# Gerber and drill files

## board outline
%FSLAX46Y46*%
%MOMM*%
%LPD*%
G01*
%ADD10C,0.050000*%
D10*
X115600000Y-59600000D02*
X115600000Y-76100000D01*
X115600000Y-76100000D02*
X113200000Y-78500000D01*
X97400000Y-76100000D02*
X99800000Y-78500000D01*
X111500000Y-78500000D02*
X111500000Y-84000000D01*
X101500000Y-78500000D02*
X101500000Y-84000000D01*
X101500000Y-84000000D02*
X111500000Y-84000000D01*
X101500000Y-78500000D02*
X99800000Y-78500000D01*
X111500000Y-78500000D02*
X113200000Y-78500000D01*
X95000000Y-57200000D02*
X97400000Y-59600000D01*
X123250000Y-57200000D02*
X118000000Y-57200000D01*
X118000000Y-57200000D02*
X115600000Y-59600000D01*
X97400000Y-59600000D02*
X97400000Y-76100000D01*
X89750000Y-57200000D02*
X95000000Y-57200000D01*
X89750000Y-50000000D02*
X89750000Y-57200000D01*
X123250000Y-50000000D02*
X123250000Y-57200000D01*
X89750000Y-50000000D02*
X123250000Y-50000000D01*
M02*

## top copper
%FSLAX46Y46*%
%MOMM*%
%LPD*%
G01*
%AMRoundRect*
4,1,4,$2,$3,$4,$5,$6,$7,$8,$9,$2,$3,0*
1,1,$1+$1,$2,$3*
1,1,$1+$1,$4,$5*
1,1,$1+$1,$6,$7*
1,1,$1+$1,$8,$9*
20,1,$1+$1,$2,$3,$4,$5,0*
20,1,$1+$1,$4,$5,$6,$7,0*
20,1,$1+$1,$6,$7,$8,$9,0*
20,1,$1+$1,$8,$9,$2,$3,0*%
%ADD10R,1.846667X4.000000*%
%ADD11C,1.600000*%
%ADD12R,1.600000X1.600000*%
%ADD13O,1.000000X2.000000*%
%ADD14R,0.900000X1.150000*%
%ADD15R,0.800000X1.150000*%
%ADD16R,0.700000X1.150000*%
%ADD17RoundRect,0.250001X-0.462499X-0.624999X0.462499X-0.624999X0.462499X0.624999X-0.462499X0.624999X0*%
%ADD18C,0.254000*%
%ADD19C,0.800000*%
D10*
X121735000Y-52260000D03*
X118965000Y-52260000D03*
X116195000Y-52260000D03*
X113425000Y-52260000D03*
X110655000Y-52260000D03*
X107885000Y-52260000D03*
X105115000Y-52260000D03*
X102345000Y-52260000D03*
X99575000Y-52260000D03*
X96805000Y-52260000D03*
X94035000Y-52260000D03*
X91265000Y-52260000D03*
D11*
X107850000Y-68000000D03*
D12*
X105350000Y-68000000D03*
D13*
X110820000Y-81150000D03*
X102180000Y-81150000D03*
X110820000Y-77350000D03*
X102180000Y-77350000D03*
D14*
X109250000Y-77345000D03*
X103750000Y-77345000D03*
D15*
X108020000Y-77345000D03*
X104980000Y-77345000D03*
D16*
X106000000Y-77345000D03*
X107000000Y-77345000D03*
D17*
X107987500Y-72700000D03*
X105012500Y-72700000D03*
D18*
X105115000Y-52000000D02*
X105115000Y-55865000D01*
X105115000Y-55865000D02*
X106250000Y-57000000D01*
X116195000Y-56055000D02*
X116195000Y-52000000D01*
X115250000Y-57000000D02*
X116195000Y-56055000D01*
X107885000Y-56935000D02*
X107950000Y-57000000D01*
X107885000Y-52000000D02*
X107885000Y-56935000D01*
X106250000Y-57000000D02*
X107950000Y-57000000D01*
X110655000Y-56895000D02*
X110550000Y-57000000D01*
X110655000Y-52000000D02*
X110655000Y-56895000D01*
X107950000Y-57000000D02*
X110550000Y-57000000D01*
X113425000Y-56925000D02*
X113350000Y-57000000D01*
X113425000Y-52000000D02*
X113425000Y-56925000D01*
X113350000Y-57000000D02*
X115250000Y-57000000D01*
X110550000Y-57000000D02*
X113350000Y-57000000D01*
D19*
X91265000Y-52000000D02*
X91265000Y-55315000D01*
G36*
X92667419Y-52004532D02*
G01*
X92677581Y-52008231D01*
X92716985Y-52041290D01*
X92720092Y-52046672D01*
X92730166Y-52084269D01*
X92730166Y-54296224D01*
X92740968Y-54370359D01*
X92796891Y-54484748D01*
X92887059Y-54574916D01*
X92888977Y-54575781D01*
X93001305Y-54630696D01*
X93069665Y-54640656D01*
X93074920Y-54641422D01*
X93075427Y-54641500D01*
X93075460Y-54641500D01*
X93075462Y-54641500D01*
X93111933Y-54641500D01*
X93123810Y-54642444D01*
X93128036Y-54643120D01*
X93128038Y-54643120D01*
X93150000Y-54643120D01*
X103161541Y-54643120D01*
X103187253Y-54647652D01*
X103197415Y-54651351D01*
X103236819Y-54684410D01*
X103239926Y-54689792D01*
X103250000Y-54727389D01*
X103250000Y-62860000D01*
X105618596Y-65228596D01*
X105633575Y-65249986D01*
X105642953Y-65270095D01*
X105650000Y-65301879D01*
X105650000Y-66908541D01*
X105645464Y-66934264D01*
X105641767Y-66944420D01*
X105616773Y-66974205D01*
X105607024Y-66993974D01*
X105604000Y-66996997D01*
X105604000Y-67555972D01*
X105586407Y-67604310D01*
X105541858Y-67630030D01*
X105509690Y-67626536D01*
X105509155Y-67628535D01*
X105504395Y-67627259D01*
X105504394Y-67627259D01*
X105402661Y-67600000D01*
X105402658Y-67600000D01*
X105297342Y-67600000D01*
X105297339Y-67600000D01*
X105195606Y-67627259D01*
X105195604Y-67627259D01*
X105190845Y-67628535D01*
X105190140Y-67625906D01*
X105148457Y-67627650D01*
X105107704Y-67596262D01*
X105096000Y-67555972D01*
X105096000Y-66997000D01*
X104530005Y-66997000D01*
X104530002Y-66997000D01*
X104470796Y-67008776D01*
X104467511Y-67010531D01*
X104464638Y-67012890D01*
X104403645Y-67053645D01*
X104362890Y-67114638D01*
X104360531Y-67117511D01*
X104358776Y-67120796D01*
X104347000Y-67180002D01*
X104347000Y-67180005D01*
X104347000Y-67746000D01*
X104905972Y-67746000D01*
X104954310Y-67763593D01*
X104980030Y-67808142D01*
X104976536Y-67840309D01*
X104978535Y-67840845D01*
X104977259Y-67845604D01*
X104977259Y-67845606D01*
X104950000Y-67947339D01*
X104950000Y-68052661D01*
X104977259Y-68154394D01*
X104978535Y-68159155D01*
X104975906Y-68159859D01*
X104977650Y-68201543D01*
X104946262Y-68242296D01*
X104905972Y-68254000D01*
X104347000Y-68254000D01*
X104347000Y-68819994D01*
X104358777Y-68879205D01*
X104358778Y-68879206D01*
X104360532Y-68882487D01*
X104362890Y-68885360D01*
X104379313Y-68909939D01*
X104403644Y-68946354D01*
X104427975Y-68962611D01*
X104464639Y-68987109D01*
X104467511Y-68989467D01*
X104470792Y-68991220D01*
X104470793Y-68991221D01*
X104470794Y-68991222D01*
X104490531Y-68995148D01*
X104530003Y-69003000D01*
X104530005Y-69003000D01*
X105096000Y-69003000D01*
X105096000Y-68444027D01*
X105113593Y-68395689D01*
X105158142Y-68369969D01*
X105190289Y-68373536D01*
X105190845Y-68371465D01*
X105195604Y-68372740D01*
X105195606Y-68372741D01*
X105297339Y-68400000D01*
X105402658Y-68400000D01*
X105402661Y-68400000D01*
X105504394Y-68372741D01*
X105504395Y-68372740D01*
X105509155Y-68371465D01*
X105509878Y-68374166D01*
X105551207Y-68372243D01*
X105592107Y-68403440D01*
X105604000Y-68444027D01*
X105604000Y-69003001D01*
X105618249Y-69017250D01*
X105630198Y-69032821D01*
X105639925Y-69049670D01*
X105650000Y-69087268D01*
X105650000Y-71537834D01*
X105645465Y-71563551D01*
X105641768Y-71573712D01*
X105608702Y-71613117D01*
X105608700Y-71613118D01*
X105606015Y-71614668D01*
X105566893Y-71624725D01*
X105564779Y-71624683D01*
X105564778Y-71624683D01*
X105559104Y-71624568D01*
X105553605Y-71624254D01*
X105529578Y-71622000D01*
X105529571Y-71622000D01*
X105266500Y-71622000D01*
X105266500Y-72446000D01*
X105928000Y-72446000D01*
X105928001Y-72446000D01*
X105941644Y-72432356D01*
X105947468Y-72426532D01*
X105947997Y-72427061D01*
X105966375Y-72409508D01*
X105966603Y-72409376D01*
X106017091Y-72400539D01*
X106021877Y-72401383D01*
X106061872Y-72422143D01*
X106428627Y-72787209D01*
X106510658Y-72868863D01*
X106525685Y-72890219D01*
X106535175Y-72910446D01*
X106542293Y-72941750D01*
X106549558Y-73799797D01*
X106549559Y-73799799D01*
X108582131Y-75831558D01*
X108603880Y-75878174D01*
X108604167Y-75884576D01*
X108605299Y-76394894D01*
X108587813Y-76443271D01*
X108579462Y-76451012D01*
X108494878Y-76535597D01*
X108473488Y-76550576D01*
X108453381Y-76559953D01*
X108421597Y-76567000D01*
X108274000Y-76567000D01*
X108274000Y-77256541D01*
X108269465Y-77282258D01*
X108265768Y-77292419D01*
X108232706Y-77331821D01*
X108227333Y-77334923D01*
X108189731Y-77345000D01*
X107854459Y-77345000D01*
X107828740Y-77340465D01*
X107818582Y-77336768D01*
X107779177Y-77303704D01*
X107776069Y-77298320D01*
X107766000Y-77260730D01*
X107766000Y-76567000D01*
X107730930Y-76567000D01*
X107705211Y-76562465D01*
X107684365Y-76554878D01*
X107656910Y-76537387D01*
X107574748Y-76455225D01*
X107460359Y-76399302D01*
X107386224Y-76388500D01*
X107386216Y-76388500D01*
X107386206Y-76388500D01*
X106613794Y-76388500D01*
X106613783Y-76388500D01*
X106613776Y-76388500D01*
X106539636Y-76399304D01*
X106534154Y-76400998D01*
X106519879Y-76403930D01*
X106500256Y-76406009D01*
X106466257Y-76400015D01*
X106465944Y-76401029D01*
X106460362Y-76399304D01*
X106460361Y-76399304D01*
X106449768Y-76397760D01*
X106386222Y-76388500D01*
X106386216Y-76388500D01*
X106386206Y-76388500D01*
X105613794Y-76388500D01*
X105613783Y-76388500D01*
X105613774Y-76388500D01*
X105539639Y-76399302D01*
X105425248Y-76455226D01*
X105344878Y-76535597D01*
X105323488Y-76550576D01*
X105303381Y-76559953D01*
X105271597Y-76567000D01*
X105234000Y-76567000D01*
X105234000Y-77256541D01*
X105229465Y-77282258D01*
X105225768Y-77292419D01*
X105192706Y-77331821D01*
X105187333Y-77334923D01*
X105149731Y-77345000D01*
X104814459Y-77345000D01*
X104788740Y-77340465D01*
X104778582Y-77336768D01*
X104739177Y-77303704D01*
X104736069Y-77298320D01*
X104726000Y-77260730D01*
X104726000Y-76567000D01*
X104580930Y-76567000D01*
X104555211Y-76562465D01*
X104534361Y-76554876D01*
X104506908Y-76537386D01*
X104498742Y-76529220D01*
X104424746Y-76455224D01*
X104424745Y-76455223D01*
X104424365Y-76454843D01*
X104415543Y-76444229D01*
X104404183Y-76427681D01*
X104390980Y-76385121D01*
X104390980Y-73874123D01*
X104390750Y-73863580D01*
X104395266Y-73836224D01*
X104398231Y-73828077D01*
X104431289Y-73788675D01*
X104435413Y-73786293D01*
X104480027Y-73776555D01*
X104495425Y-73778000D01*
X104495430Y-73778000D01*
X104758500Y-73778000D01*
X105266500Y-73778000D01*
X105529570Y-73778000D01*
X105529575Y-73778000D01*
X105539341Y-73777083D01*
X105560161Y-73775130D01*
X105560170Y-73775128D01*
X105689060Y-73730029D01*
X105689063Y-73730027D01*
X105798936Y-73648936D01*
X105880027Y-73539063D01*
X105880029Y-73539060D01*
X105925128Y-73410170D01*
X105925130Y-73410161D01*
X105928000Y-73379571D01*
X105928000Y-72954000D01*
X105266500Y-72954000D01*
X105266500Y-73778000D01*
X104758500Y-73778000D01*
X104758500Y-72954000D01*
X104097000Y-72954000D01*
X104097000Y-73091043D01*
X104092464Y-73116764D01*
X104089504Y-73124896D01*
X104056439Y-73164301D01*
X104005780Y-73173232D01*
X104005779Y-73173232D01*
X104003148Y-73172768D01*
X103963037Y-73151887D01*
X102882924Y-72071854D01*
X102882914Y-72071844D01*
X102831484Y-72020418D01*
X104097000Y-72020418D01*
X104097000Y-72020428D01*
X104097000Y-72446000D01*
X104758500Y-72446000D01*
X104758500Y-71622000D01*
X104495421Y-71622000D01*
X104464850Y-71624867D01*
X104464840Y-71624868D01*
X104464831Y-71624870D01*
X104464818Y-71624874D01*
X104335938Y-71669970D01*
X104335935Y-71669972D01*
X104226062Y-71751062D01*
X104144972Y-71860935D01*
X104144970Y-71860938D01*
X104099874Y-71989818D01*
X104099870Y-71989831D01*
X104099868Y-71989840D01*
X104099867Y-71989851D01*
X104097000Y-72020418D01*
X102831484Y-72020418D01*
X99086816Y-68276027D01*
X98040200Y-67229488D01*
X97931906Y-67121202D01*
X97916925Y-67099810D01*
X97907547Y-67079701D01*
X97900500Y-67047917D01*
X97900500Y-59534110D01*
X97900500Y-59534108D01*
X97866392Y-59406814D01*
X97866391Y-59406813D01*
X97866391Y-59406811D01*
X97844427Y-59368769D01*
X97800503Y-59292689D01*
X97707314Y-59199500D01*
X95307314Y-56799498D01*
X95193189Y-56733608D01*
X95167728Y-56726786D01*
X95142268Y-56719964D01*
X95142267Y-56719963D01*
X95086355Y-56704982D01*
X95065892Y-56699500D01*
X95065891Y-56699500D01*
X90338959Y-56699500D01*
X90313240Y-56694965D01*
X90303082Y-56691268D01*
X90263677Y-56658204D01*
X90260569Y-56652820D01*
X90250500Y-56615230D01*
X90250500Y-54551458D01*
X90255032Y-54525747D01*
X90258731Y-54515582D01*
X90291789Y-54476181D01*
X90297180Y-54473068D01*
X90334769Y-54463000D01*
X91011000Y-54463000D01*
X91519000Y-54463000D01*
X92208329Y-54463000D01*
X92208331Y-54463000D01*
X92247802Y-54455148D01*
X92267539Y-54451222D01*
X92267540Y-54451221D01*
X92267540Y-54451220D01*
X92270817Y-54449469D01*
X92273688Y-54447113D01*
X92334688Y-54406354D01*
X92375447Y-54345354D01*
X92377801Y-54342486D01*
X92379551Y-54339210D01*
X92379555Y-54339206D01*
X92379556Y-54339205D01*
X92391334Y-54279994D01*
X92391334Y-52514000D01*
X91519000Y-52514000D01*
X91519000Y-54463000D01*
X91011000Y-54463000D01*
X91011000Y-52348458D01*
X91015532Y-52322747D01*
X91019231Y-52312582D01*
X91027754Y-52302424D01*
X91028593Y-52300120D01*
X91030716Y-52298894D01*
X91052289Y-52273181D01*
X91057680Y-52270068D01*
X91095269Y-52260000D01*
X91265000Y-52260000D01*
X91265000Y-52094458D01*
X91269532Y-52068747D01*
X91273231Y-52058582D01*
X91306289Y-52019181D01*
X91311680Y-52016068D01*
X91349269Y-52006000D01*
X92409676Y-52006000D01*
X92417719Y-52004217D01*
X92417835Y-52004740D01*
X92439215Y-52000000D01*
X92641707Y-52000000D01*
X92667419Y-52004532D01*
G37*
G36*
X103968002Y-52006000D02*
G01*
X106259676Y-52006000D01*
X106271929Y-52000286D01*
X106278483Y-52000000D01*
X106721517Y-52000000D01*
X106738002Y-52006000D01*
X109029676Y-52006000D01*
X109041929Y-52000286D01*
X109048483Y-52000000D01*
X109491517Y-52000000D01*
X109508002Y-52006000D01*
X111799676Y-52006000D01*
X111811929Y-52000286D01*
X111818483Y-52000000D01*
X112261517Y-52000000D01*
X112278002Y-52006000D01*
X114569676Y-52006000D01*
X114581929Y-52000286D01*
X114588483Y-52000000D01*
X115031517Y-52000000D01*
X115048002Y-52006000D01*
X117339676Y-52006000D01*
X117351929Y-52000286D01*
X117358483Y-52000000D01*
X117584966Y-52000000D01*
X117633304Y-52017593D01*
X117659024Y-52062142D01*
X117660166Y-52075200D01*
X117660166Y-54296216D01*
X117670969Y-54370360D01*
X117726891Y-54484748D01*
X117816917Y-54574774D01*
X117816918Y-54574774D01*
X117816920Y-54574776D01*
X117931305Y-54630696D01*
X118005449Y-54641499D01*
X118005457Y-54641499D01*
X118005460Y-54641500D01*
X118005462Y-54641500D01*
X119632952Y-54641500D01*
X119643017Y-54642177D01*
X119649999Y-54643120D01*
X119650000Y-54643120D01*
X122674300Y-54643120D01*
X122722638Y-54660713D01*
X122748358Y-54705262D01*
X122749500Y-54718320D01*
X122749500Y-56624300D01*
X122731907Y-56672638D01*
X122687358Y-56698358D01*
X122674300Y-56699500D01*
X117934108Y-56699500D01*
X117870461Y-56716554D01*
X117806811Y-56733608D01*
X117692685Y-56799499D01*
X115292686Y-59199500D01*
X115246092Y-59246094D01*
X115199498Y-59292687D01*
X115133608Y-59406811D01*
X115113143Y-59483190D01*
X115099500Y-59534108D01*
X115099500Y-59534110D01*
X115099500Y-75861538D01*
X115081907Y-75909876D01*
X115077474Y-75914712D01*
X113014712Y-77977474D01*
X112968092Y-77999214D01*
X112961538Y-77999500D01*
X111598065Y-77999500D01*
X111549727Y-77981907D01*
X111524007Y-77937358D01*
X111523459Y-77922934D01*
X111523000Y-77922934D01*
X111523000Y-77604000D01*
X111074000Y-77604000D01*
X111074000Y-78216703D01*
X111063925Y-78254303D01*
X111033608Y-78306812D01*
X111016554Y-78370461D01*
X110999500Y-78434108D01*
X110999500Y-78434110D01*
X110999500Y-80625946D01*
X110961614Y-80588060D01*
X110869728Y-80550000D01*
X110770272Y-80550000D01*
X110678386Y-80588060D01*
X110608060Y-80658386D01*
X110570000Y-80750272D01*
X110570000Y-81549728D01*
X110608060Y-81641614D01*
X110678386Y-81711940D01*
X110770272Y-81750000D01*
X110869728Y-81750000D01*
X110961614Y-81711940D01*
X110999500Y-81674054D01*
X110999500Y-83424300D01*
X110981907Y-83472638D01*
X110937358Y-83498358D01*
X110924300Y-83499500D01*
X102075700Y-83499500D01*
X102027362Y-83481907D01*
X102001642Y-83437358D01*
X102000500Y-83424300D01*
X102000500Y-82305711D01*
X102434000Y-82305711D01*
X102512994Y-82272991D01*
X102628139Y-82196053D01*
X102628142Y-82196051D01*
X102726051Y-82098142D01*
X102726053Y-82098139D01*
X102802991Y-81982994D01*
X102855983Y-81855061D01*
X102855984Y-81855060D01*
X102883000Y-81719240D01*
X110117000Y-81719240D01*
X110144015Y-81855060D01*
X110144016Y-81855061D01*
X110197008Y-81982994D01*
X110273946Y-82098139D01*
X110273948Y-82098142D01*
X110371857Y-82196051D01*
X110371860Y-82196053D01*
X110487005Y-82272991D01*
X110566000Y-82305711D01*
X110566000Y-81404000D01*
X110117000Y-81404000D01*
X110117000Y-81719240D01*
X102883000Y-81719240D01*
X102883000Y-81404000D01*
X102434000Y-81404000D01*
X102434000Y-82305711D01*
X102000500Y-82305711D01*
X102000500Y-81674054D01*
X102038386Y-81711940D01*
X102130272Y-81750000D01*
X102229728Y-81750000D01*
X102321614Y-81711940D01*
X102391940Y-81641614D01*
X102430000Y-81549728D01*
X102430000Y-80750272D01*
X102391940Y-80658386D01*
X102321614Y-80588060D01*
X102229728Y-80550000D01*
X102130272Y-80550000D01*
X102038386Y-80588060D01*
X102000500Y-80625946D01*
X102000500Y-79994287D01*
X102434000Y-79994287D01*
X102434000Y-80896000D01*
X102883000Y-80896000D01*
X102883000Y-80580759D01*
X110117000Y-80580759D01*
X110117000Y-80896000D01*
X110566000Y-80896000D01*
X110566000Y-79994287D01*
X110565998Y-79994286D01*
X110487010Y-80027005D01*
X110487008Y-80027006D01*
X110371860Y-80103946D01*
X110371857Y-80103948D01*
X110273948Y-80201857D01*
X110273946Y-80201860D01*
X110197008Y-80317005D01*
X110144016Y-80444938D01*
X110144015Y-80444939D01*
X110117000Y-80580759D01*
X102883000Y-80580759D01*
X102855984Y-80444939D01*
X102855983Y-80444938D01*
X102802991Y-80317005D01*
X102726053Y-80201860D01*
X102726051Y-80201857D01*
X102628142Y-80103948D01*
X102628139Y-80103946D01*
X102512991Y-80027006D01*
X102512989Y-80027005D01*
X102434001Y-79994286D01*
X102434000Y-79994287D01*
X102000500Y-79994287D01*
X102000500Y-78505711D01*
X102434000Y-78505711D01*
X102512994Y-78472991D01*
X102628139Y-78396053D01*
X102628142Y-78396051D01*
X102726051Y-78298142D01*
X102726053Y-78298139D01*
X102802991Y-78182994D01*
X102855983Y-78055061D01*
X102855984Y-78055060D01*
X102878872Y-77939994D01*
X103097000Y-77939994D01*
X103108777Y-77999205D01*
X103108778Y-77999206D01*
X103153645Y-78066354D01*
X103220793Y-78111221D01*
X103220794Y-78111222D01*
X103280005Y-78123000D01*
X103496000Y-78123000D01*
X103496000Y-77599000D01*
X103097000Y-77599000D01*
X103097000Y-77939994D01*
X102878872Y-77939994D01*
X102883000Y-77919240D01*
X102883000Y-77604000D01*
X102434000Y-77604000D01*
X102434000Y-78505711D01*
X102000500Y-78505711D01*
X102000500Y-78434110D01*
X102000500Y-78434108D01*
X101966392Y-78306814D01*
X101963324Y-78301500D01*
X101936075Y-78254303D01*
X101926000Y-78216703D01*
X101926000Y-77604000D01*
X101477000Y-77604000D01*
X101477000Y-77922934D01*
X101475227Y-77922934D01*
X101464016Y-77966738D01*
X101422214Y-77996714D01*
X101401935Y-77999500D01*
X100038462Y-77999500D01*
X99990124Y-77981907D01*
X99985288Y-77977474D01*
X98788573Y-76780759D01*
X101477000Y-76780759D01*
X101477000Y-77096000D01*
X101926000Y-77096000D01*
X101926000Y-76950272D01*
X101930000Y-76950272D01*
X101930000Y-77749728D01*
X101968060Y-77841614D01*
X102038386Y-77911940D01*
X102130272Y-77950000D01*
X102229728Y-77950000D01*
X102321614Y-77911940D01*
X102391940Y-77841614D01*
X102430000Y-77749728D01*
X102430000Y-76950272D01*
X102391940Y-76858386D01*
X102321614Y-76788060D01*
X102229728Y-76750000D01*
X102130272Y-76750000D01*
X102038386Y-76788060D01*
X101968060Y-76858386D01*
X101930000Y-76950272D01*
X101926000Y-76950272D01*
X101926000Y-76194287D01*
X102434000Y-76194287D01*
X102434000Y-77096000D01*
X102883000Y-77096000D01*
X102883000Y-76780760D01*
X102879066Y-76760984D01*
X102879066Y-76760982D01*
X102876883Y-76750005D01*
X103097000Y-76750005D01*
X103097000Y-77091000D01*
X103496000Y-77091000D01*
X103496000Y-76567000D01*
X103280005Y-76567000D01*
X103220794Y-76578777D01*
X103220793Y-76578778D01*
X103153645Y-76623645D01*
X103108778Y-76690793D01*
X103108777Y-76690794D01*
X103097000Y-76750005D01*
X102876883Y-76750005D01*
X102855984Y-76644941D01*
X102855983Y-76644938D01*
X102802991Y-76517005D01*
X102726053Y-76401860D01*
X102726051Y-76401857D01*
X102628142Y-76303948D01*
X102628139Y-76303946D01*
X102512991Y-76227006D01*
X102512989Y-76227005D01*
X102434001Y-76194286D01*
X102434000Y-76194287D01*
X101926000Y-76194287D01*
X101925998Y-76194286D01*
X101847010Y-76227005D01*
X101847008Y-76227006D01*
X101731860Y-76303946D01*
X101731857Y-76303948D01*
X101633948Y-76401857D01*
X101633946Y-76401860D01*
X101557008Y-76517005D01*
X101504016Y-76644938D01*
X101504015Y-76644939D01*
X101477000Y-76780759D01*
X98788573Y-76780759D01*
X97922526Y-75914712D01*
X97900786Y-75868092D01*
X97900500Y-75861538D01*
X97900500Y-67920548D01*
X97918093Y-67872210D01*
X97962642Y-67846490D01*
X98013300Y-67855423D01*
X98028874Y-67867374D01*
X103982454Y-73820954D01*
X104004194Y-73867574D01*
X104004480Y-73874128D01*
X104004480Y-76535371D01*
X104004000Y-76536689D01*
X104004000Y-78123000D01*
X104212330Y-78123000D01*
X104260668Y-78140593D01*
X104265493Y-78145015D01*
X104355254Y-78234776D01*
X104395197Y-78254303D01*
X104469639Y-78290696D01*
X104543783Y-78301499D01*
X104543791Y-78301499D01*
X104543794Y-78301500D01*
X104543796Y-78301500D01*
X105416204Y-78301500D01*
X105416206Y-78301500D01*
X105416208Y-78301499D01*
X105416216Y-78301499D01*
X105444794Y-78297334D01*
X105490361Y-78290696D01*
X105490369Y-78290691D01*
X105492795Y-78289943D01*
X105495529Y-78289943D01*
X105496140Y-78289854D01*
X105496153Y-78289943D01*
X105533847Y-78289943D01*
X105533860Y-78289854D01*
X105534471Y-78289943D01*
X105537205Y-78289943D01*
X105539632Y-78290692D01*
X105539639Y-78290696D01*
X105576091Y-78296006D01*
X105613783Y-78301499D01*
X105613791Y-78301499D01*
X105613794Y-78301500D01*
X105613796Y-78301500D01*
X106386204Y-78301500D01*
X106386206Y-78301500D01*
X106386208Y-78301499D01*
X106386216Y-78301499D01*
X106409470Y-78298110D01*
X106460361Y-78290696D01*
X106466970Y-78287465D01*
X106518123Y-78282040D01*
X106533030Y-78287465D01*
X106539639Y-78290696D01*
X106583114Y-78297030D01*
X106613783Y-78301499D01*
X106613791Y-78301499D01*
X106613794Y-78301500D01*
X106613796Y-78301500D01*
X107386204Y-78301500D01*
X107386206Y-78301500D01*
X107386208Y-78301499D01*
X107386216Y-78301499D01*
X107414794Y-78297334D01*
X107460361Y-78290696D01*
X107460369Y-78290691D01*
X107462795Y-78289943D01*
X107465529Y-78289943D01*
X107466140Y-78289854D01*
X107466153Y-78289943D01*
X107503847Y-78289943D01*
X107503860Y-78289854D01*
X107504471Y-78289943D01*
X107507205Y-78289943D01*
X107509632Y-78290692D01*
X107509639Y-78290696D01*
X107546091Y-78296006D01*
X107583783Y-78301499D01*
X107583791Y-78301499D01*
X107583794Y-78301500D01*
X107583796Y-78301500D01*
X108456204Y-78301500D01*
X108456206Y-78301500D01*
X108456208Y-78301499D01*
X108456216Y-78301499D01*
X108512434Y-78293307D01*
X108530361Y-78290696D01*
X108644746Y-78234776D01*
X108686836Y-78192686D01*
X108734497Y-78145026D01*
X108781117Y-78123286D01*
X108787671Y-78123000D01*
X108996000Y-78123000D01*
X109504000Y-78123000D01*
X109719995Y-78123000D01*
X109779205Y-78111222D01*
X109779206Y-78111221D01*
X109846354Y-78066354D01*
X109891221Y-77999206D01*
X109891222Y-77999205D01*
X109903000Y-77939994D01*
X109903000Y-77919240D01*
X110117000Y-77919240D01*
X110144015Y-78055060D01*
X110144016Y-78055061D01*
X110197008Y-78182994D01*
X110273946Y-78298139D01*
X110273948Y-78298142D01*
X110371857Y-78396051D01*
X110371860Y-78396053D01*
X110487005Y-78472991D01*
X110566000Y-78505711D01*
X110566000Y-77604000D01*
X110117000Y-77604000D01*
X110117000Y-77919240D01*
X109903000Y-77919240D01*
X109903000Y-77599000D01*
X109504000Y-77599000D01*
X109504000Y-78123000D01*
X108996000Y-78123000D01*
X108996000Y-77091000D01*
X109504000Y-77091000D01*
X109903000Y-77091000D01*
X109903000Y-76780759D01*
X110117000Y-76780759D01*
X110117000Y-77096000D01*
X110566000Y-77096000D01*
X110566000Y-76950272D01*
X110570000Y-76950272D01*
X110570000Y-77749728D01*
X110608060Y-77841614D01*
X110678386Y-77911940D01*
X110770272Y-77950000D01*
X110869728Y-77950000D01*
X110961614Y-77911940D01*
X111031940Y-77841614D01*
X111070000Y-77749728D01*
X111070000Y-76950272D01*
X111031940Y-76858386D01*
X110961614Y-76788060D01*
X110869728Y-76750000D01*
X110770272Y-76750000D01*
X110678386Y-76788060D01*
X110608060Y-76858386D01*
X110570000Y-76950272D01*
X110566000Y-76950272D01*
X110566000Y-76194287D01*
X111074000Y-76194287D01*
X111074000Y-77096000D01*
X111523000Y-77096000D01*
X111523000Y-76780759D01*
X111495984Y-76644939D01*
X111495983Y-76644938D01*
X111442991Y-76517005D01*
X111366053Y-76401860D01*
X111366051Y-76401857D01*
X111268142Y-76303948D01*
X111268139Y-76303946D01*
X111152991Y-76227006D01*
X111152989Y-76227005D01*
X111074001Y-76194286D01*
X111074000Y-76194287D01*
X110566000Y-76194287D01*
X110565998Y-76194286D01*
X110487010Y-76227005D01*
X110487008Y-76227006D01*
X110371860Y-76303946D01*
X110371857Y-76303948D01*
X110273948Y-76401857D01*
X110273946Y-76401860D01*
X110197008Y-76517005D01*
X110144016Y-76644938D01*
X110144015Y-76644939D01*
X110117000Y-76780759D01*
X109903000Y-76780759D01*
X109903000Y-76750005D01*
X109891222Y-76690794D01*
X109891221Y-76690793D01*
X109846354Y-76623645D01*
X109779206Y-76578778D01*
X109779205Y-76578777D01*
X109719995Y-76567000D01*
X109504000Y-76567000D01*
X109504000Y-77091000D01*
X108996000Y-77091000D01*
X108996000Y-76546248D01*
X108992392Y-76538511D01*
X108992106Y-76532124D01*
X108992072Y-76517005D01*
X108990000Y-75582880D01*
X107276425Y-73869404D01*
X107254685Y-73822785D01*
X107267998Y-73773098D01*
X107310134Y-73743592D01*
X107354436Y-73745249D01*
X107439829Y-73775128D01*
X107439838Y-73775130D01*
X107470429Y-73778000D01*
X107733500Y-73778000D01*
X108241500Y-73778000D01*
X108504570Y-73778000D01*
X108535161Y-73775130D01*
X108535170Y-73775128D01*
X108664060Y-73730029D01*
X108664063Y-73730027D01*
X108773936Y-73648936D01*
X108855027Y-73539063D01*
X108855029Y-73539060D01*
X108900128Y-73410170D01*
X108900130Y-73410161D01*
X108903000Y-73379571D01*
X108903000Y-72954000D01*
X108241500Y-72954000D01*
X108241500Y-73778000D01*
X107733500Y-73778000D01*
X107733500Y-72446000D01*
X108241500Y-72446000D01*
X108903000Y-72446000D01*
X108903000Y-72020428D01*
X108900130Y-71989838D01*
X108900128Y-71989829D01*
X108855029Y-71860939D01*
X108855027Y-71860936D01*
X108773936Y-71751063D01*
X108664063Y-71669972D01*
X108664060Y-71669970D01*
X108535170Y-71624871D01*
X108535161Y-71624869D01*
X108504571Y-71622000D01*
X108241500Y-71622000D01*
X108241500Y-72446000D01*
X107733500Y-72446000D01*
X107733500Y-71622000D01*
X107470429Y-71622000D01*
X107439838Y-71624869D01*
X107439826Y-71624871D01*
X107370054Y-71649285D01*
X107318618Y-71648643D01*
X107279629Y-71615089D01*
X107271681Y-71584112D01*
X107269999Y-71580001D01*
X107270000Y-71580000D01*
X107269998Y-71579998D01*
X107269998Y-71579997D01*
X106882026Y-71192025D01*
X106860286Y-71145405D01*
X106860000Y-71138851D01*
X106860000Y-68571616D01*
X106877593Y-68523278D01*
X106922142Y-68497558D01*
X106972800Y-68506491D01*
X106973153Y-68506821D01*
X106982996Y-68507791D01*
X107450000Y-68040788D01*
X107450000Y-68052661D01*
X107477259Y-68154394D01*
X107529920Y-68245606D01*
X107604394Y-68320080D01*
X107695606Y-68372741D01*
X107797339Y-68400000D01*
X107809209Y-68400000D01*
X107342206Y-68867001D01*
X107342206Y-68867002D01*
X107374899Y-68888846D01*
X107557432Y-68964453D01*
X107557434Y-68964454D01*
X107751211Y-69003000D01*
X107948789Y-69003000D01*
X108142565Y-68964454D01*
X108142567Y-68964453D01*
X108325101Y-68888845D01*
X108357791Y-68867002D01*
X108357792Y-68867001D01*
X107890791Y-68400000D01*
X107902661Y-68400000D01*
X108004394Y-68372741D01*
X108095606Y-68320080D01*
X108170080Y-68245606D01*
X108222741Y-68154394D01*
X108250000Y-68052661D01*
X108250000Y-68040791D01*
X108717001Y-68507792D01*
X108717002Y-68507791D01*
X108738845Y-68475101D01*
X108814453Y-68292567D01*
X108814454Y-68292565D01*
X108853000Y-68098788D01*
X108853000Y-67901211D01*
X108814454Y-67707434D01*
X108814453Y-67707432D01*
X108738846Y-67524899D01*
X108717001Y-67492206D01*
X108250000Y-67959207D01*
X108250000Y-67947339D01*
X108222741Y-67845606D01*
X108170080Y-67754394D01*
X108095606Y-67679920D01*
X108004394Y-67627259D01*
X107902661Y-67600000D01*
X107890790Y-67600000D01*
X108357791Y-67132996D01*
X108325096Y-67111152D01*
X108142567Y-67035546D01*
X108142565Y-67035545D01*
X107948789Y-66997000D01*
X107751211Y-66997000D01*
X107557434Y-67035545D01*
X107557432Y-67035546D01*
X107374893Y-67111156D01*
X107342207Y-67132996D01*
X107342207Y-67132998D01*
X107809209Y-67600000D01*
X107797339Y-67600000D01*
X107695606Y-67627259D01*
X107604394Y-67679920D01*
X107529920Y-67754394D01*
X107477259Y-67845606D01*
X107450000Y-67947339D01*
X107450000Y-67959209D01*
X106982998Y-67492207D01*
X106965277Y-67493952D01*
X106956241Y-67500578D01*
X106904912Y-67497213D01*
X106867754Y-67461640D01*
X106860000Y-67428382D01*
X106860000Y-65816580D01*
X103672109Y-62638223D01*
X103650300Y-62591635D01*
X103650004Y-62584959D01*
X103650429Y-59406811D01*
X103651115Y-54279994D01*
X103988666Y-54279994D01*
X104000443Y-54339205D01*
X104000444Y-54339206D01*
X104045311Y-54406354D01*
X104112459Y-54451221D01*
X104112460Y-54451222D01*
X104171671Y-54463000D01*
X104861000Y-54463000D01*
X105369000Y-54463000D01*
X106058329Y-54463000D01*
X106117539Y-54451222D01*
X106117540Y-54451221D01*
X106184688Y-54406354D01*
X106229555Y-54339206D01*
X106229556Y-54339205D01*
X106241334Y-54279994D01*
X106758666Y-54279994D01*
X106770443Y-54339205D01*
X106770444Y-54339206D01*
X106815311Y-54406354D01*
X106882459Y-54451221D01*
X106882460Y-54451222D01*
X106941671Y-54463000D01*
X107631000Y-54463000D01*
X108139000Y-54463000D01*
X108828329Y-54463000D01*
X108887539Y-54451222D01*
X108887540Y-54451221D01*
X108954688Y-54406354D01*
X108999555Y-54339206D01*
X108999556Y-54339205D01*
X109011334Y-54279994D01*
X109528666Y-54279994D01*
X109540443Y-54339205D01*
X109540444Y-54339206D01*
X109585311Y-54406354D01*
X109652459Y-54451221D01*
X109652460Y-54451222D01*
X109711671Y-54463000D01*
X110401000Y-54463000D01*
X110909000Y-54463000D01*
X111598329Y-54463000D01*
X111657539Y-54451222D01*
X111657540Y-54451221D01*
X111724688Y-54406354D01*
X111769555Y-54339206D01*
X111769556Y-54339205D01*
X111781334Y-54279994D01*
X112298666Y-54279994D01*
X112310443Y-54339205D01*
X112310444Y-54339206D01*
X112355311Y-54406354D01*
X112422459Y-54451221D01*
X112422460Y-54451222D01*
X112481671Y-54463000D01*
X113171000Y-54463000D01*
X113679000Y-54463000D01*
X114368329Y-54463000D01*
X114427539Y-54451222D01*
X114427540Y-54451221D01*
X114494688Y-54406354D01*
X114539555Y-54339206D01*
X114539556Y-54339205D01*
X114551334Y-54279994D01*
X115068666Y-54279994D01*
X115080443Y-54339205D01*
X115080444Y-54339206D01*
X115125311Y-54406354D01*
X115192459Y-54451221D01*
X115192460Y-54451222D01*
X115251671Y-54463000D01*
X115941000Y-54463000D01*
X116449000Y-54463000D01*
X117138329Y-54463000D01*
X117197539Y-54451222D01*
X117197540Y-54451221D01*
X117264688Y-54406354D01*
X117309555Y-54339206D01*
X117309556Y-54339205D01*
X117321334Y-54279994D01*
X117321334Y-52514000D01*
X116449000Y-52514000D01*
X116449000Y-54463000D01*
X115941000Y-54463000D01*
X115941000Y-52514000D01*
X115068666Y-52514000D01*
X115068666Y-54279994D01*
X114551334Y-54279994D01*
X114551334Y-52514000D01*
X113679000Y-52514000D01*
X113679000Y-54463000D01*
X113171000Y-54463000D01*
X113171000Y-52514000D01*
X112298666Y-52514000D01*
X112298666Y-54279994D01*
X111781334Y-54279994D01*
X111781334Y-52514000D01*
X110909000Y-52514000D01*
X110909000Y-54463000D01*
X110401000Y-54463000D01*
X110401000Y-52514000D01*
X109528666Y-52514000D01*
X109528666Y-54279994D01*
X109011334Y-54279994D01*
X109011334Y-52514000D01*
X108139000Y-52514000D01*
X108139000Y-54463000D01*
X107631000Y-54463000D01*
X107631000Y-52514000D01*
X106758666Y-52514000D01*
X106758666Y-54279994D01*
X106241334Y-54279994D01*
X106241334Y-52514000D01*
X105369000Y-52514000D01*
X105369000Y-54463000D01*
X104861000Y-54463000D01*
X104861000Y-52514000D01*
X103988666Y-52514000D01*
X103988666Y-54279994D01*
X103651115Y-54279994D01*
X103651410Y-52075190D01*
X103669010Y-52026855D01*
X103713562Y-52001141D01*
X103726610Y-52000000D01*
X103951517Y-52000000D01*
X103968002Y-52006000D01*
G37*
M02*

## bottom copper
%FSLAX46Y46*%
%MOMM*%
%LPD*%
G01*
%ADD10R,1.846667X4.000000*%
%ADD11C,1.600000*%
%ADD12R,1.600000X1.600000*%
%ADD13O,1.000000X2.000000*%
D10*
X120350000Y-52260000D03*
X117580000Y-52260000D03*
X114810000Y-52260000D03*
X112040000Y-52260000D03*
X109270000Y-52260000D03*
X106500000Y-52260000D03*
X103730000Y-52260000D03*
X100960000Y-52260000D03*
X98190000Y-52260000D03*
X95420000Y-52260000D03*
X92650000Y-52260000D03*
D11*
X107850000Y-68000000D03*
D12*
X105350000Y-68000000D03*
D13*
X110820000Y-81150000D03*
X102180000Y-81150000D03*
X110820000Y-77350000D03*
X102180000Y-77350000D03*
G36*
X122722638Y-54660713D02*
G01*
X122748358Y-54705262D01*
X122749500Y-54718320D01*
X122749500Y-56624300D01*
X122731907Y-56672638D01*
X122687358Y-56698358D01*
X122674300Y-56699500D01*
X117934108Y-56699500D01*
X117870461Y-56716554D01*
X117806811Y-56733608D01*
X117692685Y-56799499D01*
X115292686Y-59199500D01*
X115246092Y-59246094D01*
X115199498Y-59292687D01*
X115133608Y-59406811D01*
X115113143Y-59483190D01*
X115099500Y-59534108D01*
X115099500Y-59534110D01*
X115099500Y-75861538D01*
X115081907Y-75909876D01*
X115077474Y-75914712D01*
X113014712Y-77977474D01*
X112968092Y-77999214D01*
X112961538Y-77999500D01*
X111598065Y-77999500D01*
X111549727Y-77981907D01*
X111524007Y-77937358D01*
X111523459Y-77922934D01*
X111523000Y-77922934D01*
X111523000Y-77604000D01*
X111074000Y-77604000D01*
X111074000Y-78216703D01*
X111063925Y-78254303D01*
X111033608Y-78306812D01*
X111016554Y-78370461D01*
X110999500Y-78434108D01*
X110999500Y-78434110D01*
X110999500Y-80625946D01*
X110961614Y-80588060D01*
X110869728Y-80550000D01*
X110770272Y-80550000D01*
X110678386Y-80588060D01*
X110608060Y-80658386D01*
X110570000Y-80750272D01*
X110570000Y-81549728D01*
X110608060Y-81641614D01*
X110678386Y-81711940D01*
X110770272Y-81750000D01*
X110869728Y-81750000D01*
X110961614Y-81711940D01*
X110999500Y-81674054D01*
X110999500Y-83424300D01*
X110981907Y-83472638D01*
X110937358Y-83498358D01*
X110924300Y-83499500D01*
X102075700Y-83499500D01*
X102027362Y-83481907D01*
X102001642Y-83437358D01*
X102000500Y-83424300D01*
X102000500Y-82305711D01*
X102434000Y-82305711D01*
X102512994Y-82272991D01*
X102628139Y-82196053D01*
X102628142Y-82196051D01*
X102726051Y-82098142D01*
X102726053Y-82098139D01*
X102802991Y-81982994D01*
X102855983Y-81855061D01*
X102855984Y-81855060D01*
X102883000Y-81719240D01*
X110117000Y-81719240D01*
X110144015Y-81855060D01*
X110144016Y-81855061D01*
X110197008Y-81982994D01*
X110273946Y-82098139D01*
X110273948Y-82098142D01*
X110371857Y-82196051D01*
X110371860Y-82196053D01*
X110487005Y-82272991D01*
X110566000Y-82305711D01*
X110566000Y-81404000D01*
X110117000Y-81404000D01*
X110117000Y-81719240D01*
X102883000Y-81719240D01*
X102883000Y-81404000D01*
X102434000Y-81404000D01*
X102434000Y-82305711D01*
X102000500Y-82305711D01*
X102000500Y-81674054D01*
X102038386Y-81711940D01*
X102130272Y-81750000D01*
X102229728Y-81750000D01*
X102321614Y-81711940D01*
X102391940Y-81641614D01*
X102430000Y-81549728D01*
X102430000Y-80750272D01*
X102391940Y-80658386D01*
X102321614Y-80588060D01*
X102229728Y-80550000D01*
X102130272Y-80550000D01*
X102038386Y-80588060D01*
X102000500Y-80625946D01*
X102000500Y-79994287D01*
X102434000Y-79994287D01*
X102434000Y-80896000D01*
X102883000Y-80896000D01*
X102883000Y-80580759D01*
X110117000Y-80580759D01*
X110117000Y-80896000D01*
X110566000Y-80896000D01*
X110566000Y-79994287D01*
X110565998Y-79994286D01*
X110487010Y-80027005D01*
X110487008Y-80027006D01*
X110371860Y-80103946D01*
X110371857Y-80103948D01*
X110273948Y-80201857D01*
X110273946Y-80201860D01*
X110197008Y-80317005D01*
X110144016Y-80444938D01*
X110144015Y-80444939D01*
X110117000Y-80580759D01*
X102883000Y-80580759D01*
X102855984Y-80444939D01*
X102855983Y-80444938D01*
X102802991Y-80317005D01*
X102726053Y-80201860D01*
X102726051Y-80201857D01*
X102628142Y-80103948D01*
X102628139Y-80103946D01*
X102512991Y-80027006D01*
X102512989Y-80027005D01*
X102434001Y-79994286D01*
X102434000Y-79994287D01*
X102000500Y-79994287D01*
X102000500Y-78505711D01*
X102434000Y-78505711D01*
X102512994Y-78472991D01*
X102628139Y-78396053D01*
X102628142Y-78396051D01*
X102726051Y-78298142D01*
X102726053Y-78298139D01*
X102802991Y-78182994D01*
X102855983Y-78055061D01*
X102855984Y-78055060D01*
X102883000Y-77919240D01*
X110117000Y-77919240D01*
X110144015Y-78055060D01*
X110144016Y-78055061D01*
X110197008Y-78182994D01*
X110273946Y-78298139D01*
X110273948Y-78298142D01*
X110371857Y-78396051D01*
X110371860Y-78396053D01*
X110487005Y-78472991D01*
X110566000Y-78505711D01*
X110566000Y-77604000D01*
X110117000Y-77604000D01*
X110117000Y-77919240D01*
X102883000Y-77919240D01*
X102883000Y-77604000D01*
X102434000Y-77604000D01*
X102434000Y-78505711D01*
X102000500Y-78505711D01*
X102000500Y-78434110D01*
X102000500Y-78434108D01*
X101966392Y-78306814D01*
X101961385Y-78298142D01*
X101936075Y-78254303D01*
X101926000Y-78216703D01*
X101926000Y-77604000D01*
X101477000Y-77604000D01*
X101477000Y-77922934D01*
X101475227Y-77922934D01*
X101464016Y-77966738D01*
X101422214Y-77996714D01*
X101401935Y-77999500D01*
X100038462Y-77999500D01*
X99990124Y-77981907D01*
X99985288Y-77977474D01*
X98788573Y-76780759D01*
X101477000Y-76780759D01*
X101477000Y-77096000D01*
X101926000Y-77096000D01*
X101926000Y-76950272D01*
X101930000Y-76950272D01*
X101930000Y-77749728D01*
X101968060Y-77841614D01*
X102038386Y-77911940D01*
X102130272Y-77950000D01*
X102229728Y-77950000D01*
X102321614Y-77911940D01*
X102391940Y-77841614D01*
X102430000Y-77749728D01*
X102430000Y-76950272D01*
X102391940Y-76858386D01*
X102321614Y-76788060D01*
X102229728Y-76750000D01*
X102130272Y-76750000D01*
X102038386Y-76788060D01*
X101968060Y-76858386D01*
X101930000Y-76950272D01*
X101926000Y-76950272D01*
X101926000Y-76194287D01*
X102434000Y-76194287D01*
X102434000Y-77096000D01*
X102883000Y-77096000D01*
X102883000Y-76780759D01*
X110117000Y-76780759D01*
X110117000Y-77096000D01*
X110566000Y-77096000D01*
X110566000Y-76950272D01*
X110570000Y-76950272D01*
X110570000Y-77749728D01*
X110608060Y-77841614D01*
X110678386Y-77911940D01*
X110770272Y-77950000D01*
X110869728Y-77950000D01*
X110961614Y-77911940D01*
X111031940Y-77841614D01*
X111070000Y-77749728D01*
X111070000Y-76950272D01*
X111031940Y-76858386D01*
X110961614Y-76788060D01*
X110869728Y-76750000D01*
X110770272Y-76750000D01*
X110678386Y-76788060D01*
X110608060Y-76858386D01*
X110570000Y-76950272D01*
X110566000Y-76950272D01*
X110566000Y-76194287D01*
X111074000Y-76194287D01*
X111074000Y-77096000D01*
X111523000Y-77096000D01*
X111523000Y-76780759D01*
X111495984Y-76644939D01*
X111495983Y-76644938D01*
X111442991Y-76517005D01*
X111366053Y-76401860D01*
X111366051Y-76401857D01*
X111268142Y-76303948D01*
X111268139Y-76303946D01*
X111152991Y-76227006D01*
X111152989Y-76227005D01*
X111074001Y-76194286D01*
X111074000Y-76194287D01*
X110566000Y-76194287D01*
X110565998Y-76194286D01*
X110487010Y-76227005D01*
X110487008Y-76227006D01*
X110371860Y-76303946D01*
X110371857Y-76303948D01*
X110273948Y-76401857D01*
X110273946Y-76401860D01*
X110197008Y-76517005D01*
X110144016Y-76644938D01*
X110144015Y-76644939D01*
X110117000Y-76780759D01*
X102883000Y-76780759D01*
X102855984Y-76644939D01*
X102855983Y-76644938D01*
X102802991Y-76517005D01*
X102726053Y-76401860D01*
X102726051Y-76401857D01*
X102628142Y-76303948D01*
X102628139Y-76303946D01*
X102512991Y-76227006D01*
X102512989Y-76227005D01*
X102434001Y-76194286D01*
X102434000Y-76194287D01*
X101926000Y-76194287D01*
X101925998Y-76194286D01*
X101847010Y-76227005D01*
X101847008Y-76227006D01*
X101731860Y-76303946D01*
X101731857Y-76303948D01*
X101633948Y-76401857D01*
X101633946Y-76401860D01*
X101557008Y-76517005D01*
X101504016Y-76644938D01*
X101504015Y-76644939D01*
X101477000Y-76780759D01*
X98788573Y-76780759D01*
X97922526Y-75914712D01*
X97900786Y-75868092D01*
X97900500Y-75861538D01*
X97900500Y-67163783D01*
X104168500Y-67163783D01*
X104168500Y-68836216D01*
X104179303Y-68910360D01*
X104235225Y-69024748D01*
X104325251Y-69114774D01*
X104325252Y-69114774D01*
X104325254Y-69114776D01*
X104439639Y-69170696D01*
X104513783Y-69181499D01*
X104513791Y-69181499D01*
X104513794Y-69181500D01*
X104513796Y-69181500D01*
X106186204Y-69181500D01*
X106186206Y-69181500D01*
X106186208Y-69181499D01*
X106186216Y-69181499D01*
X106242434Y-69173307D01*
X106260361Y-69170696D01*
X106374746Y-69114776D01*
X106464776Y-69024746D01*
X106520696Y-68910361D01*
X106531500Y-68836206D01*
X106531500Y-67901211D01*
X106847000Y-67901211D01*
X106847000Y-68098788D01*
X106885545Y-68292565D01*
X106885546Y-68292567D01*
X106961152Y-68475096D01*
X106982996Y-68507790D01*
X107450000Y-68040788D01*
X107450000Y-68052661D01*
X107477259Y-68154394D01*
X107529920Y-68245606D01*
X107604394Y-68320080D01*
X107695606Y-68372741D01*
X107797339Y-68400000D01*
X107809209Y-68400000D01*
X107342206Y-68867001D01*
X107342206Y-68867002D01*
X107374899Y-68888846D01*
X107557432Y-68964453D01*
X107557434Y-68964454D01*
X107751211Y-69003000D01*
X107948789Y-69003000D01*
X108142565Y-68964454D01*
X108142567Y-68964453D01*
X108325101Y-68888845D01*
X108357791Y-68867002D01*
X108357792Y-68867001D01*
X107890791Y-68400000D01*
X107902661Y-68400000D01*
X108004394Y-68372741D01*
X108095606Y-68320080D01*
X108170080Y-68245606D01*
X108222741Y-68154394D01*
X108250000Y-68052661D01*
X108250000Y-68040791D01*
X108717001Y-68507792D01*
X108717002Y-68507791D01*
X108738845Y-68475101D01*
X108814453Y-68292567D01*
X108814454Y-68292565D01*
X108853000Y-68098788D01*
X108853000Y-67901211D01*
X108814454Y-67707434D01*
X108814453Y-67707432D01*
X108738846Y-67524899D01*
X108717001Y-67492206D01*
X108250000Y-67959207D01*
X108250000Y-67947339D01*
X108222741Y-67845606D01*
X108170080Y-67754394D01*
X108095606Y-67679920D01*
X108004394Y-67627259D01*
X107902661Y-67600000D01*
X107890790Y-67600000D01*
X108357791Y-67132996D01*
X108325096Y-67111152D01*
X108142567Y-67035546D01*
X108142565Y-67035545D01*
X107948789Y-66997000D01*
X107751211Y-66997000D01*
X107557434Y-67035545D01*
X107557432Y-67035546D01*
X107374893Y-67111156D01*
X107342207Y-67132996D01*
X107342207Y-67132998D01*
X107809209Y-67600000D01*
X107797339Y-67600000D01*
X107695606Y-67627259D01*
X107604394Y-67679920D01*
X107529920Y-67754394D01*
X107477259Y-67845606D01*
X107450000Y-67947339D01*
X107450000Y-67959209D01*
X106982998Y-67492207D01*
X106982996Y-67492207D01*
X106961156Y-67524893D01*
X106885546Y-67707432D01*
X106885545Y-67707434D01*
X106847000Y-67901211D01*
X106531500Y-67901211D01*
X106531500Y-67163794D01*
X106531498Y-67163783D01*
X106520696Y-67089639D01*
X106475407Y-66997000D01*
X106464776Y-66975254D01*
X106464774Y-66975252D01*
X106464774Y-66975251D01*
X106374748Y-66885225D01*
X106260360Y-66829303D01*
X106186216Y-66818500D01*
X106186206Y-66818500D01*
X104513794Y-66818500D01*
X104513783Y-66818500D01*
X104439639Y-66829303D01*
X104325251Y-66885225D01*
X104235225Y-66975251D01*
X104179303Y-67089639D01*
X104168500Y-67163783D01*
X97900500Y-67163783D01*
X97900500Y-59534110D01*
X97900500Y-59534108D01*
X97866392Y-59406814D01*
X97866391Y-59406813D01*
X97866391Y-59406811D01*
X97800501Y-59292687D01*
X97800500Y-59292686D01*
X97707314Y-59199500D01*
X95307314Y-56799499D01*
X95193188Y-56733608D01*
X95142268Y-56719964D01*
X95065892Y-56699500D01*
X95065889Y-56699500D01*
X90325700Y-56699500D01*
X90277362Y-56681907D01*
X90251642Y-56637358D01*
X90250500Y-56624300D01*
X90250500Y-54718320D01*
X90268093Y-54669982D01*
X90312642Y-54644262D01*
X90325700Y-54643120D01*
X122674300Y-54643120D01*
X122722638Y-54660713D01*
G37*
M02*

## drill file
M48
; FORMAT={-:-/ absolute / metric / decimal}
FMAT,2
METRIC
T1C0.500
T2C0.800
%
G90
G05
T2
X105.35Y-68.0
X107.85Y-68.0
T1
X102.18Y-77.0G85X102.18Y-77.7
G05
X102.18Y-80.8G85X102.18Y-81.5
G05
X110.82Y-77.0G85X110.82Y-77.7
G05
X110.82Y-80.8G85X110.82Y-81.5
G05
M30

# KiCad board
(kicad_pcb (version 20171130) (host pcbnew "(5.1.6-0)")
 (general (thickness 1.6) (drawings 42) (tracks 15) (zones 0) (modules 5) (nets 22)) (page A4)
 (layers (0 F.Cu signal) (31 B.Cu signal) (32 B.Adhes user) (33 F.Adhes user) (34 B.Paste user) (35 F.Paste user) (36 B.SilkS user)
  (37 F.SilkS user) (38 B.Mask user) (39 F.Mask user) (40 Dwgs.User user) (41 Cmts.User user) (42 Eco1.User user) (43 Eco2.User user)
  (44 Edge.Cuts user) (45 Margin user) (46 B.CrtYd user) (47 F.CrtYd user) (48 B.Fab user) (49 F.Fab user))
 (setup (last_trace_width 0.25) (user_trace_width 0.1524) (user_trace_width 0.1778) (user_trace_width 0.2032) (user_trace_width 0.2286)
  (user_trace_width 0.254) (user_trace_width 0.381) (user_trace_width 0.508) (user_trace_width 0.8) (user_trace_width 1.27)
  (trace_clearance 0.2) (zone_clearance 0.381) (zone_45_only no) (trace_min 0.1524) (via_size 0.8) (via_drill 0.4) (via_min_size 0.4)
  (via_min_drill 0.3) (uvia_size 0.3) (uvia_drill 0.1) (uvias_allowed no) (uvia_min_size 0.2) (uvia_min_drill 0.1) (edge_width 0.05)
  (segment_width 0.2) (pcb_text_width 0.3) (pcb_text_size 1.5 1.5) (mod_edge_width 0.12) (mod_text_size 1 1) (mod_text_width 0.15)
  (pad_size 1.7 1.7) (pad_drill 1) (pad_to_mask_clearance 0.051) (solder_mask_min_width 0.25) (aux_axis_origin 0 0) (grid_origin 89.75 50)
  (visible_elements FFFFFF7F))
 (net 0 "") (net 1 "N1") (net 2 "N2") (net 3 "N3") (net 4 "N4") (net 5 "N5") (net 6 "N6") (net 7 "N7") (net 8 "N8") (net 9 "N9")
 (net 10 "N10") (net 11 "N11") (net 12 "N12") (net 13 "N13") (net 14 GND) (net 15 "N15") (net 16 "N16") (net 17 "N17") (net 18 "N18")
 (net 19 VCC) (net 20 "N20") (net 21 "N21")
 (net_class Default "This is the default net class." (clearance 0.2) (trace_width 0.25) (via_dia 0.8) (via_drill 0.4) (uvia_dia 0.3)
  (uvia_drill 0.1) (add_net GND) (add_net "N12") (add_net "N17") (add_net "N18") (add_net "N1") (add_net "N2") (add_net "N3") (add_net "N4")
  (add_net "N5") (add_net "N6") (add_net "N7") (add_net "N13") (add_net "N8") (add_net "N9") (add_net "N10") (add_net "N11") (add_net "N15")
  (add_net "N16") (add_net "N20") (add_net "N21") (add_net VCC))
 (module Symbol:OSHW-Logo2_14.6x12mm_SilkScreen (layer B.Cu) (at 106.5 63.75 180)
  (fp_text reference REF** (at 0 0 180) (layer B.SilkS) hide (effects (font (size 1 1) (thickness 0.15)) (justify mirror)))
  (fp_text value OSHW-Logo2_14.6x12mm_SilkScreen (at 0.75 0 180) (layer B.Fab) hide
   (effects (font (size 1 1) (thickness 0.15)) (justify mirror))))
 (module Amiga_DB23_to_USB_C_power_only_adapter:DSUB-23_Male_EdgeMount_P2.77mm (layer F.Cu) (at 106.5 52 180)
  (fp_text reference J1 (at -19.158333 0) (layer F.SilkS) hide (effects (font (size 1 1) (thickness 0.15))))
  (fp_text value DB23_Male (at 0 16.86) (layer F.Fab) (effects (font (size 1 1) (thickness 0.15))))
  (pad 13 smd rect (at -13.85 0 180) (size 1.846667 4) (drill (offset 0 -0.26)) (layers B.Cu B.Paste B.Mask) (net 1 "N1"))
  (pad 14 smd rect (at -11.08 0 180) (size 1.846667 4) (drill (offset 0 -0.26)) (layers B.Cu B.Paste B.Mask) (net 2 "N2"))
  (pad 15 smd rect (at -8.31 0 180) (size 1.846667 4) (drill (offset 0 -0.26)) (layers B.Cu B.Paste B.Mask) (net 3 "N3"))
  (pad 16 smd rect (at -5.54 0 180) (size 1.846667 4) (drill (offset 0 -0.26)) (layers B.Cu B.Paste B.Mask) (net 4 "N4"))
  (pad 17 smd rect (at -2.77 0 180) (size 1.846667 4) (drill (offset 0 -0.26)) (layers B.Cu B.Paste B.Mask) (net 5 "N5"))
  (pad 18 smd rect (at 0 0 180) (size 1.846667 4) (drill (offset 0 -0.26)) (layers B.Cu B.Paste B.Mask) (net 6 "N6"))
  (pad 19 smd rect (at 2.77 0 180) (size 1.846667 4) (drill (offset 0 -0.26)) (layers B.Cu B.Paste B.Mask) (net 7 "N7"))
  (pad 20 smd rect (at 5.54 0 180) (size 1.846667 4) (drill (offset 0 -0.26)) (layers B.Cu B.Paste B.Mask) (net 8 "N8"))
  (pad 21 smd rect (at 8.31 0 180) (size 1.846667 4) (drill (offset 0 -0.26)) (layers B.Cu B.Paste B.Mask) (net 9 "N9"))
  (pad 22 smd rect (at 11.08 0 180) (size 1.846667 4) (drill (offset 0 -0.26)) (layers B.Cu B.Paste B.Mask) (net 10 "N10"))
  (pad 23 smd rect (at 13.85 0 180) (size 1.846667 4) (drill (offset 0 -0.26)) (layers B.Cu B.Paste B.Mask) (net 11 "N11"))
  (pad 1 smd rect (at -15.235 0 180) (size 1.846667 4) (drill (offset 0 -0.26)) (layers F.Cu F.Paste F.Mask) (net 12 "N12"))
  (pad 2 smd rect (at -12.465 0 180) (size 1.846667 4) (drill (offset 0 -0.26)) (layers F.Cu F.Paste F.Mask) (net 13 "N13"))
  (pad 3 smd rect (at -9.695 0 180) (size 1.846667 4) (drill (offset 0 -0.26)) (layers F.Cu F.Paste F.Mask) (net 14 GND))
  (pad 4 smd rect (at -6.925 0 180) (size 1.846667 4) (drill (offset 0 -0.26)) (layers F.Cu F.Paste F.Mask) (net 14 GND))
  (pad 5 smd rect (at -4.155 0 180) (size 1.846667 4) (drill (offset 0 -0.26)) (layers F.Cu F.Paste F.Mask) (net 14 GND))
  (pad 6 smd rect (at -1.385 0 180) (size 1.846667 4) (drill (offset 0 -0.26)) (layers F.Cu F.Paste F.Mask) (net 14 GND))
  (pad 7 smd rect (at 1.385 0 180) (size 1.846667 4) (drill (offset 0 -0.26)) (layers F.Cu F.Paste F.Mask) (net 14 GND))
  (pad 8 smd rect (at 4.155 0 180) (size 1.846667 4) (drill (offset 0 -0.26)) (layers F.Cu F.Paste F.Mask) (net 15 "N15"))
  (pad 9 smd rect (at 6.925 0 180) (size 1.846667 4) (drill (offset 0 -0.26)) (layers F.Cu F.Paste F.Mask) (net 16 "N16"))
  (pad 10 smd rect (at 9.695 0 180) (size 1.846667 4) (drill (offset 0 -0.26)) (layers F.Cu F.Paste F.Mask) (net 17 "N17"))
  (pad 11 smd rect (at 12.465 0 180) (size 1.846667 4) (drill (offset 0 -0.26)) (layers F.Cu F.Paste F.Mask) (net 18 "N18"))
  (pad 12 smd rect (at 15.235 0 180) (size 1.846667 4) (drill (offset 0 -0.26)) (layers F.Cu F.Paste F.Mask) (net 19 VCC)))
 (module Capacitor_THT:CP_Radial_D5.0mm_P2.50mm (layer F.Cu) (at 105.35 68)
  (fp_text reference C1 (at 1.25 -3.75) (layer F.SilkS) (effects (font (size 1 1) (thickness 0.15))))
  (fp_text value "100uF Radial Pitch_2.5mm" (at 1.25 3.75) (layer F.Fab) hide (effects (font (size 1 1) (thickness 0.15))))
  (pad 2 thru_hole circle (at 2.5 0) (size 1.6 1.6) (drill 0.8) (layers *.Cu *.Mask) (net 14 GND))
  (pad 1 thru_hole rect (at 0 0) (size 1.6 1.6) (drill 0.8) (layers *.Cu *.Mask) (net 19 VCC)))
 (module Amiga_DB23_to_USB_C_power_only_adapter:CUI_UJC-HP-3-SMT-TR (layer F.Cu) (at 106.5 77.35)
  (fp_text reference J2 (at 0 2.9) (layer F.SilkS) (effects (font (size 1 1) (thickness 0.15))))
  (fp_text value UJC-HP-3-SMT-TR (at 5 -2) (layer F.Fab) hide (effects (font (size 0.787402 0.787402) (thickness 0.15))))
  (pad S4 thru_hole oval (at 4.32 3.8) (size 1 2) (drill oval 0.5 1.2) (layers *.Cu *.Mask) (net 14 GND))
  (pad S3 thru_hole oval (at -4.32 3.8) (size 1 2) (drill oval 0.5 1.2) (layers *.Cu *.Mask) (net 14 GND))
  (pad S2 thru_hole oval (at 4.32 0) (size 1 2) (drill oval 0.5 1.2) (layers *.Cu *.Mask) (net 14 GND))
  (pad S1 thru_hole oval (at -4.32 0) (size 1 2) (drill oval 0.5 1.2) (layers *.Cu *.Mask) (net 14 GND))
  (pad A12 smd rect (at 2.75 -0.005 90) (size 1.15 0.9) (layers F.Cu F.Paste F.Mask) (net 14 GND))
  (pad B12 smd rect (at -2.75 -0.005 90) (size 1.15 0.9) (layers F.Cu F.Paste F.Mask) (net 14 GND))
  (pad A9 smd rect (at 1.52 -0.005 90) (size 1.15 0.8) (layers F.Cu F.Paste F.Mask) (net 19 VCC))
  (pad B9 smd rect (at -1.52 -0.005 90) (size 1.15 0.8) (layers F.Cu F.Paste F.Mask) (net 19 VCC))
  (pad A5 smd rect (at -0.5 -0.005 90) (size 1.15 0.7) (layers F.Cu F.Paste F.Mask) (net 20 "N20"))
  (pad B5 smd rect (at 0.5 -0.005 90) (size 1.15 0.7) (layers F.Cu F.Paste F.Mask) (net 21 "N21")))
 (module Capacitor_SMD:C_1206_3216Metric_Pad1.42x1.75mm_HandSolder (layer F.Cu) (at 106.5 72.7)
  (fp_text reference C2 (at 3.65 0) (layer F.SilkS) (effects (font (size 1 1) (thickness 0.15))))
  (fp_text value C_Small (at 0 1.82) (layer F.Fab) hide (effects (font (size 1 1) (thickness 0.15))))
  (pad 2 smd roundrect (at 1.4875 0) (size 1.425 1.75) (layers F.Cu F.Paste F.Mask) (roundrect_rratio 0.175439) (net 14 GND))
  (pad 1 smd roundrect (at -1.4875 0) (size 1.425 1.75) (layers F.Cu F.Paste F.Mask) (roundrect_rratio 0.175439) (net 19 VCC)))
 (gr_line (start 115.6 59.6) (end 115.6 76.1) (layer Edge.Cuts) (width 0.05))
 (gr_line (start 115.6 76.1) (end 113.2 78.5) (layer Edge.Cuts) (width 0.05))
 (gr_line (start 97.4 76.1) (end 99.8 78.5) (layer Edge.Cuts) (width 0.05))
 (gr_line (start 111.5 78.5) (end 111.5 84) (layer Edge.Cuts) (width 0.05))
 (gr_line (start 101.5 78.5) (end 101.5 84) (layer Edge.Cuts) (width 0.05))
 (gr_line (start 101.5 84) (end 111.5 84) (layer Edge.Cuts) (width 0.05))
 (gr_line (start 101.5 78.5) (end 99.8 78.5) (layer Edge.Cuts) (width 0.05))
 (gr_line (start 111.5 78.5) (end 113.2 78.5) (layer Edge.Cuts) (width 0.05))
 (gr_line (start 95 57.2) (end 97.4 59.6) (layer Edge.Cuts) (width 0.05))
 (gr_line (start 123.25 57.2) (end 118 57.2) (layer Edge.Cuts) (width 0.05))
 (gr_line (start 118 57.2) (end 115.6 59.6) (layer Edge.Cuts) (width 0.05))
 (gr_line (start 97.4 59.6) (end 97.4 76.1) (layer Edge.Cuts) (width 0.05))
 (gr_line (start 89.75 57.2) (end 95 57.2) (layer Edge.Cuts) (width 0.05))
 (gr_line (start 89.75 50) (end 89.75 57.2) (layer Edge.Cuts) (width 0.05))
 (gr_line (start 123.25 50) (end 123.25 57.2) (layer Edge.Cuts) (width 0.05))
 (gr_line (start 89.75 50) (end 123.25 50) (layer Edge.Cuts) (width 0.05))
 (segment (start 105.115 52) (end 105.115 55.865) (width 0.254) (layer F.Cu) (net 14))
 (segment (start 105.115 55.865) (end 106.25 57) (width 0.254) (layer F.Cu) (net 14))
 (segment (start 116.195 56.055) (end 116.195 52) (width 0.254) (layer F.Cu) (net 14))
 (segment (start 115.25 57) (end 116.195 56.055) (width 0.254) (layer F.Cu) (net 14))
 (segment (start 107.885 56.935) (end 107.95 57) (width 0.254) (layer F.Cu) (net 14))
 (segment (start 107.885 52) (end 107.885 56.935) (width 0.254) (layer F.Cu) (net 14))
 (segment (start 106.25 57) (end 107.95 57) (width 0.254) (layer F.Cu) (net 14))
 (segment (start 110.655 56.895) (end 110.55 57) (width 0.254) (layer F.Cu) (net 14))
 (segment (start 110.655 52) (end 110.655 56.895) (width 0.254) (layer F.Cu) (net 14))
 (segment (start 107.95 57) (end 110.55 57) (width 0.254) (layer F.Cu) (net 14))
 (segment (start 113.425 56.925) (end 113.35 57) (width 0.254) (layer F.Cu) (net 14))
 (segment (start 113.425 52) (end 113.425 56.925) (width 0.254) (layer F.Cu) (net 14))
 (segment (start 113.35 57) (end 115.25 57) (width 0.254) (layer F.Cu) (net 14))
 (segment (start 110.55 57) (end 113.35 57) (width 0.254) (layer F.Cu) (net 14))
 (segment (start 91.265 52) (end 91.265 55.315) (width 0.8) (layer F.Cu) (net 19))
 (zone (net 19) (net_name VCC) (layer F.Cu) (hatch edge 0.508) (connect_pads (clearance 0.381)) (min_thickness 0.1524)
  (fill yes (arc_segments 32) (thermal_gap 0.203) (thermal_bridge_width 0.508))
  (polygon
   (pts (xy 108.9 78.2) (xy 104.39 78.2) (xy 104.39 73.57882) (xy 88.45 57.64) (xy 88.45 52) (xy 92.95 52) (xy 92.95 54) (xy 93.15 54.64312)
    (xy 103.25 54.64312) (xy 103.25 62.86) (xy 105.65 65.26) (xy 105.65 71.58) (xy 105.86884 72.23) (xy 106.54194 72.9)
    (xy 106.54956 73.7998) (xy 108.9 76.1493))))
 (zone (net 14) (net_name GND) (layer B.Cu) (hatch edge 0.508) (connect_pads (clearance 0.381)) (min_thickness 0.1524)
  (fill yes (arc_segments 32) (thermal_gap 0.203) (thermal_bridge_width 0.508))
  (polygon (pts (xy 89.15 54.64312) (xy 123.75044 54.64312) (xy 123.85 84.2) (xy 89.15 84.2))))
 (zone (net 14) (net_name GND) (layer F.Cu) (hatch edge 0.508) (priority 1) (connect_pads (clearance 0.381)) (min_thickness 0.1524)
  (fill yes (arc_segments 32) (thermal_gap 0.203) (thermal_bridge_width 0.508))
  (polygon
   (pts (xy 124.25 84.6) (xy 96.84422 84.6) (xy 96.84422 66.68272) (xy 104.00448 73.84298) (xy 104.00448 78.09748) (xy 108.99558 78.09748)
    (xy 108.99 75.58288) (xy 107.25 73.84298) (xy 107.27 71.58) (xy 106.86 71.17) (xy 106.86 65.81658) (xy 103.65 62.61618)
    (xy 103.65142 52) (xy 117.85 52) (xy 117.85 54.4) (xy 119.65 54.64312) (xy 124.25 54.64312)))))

